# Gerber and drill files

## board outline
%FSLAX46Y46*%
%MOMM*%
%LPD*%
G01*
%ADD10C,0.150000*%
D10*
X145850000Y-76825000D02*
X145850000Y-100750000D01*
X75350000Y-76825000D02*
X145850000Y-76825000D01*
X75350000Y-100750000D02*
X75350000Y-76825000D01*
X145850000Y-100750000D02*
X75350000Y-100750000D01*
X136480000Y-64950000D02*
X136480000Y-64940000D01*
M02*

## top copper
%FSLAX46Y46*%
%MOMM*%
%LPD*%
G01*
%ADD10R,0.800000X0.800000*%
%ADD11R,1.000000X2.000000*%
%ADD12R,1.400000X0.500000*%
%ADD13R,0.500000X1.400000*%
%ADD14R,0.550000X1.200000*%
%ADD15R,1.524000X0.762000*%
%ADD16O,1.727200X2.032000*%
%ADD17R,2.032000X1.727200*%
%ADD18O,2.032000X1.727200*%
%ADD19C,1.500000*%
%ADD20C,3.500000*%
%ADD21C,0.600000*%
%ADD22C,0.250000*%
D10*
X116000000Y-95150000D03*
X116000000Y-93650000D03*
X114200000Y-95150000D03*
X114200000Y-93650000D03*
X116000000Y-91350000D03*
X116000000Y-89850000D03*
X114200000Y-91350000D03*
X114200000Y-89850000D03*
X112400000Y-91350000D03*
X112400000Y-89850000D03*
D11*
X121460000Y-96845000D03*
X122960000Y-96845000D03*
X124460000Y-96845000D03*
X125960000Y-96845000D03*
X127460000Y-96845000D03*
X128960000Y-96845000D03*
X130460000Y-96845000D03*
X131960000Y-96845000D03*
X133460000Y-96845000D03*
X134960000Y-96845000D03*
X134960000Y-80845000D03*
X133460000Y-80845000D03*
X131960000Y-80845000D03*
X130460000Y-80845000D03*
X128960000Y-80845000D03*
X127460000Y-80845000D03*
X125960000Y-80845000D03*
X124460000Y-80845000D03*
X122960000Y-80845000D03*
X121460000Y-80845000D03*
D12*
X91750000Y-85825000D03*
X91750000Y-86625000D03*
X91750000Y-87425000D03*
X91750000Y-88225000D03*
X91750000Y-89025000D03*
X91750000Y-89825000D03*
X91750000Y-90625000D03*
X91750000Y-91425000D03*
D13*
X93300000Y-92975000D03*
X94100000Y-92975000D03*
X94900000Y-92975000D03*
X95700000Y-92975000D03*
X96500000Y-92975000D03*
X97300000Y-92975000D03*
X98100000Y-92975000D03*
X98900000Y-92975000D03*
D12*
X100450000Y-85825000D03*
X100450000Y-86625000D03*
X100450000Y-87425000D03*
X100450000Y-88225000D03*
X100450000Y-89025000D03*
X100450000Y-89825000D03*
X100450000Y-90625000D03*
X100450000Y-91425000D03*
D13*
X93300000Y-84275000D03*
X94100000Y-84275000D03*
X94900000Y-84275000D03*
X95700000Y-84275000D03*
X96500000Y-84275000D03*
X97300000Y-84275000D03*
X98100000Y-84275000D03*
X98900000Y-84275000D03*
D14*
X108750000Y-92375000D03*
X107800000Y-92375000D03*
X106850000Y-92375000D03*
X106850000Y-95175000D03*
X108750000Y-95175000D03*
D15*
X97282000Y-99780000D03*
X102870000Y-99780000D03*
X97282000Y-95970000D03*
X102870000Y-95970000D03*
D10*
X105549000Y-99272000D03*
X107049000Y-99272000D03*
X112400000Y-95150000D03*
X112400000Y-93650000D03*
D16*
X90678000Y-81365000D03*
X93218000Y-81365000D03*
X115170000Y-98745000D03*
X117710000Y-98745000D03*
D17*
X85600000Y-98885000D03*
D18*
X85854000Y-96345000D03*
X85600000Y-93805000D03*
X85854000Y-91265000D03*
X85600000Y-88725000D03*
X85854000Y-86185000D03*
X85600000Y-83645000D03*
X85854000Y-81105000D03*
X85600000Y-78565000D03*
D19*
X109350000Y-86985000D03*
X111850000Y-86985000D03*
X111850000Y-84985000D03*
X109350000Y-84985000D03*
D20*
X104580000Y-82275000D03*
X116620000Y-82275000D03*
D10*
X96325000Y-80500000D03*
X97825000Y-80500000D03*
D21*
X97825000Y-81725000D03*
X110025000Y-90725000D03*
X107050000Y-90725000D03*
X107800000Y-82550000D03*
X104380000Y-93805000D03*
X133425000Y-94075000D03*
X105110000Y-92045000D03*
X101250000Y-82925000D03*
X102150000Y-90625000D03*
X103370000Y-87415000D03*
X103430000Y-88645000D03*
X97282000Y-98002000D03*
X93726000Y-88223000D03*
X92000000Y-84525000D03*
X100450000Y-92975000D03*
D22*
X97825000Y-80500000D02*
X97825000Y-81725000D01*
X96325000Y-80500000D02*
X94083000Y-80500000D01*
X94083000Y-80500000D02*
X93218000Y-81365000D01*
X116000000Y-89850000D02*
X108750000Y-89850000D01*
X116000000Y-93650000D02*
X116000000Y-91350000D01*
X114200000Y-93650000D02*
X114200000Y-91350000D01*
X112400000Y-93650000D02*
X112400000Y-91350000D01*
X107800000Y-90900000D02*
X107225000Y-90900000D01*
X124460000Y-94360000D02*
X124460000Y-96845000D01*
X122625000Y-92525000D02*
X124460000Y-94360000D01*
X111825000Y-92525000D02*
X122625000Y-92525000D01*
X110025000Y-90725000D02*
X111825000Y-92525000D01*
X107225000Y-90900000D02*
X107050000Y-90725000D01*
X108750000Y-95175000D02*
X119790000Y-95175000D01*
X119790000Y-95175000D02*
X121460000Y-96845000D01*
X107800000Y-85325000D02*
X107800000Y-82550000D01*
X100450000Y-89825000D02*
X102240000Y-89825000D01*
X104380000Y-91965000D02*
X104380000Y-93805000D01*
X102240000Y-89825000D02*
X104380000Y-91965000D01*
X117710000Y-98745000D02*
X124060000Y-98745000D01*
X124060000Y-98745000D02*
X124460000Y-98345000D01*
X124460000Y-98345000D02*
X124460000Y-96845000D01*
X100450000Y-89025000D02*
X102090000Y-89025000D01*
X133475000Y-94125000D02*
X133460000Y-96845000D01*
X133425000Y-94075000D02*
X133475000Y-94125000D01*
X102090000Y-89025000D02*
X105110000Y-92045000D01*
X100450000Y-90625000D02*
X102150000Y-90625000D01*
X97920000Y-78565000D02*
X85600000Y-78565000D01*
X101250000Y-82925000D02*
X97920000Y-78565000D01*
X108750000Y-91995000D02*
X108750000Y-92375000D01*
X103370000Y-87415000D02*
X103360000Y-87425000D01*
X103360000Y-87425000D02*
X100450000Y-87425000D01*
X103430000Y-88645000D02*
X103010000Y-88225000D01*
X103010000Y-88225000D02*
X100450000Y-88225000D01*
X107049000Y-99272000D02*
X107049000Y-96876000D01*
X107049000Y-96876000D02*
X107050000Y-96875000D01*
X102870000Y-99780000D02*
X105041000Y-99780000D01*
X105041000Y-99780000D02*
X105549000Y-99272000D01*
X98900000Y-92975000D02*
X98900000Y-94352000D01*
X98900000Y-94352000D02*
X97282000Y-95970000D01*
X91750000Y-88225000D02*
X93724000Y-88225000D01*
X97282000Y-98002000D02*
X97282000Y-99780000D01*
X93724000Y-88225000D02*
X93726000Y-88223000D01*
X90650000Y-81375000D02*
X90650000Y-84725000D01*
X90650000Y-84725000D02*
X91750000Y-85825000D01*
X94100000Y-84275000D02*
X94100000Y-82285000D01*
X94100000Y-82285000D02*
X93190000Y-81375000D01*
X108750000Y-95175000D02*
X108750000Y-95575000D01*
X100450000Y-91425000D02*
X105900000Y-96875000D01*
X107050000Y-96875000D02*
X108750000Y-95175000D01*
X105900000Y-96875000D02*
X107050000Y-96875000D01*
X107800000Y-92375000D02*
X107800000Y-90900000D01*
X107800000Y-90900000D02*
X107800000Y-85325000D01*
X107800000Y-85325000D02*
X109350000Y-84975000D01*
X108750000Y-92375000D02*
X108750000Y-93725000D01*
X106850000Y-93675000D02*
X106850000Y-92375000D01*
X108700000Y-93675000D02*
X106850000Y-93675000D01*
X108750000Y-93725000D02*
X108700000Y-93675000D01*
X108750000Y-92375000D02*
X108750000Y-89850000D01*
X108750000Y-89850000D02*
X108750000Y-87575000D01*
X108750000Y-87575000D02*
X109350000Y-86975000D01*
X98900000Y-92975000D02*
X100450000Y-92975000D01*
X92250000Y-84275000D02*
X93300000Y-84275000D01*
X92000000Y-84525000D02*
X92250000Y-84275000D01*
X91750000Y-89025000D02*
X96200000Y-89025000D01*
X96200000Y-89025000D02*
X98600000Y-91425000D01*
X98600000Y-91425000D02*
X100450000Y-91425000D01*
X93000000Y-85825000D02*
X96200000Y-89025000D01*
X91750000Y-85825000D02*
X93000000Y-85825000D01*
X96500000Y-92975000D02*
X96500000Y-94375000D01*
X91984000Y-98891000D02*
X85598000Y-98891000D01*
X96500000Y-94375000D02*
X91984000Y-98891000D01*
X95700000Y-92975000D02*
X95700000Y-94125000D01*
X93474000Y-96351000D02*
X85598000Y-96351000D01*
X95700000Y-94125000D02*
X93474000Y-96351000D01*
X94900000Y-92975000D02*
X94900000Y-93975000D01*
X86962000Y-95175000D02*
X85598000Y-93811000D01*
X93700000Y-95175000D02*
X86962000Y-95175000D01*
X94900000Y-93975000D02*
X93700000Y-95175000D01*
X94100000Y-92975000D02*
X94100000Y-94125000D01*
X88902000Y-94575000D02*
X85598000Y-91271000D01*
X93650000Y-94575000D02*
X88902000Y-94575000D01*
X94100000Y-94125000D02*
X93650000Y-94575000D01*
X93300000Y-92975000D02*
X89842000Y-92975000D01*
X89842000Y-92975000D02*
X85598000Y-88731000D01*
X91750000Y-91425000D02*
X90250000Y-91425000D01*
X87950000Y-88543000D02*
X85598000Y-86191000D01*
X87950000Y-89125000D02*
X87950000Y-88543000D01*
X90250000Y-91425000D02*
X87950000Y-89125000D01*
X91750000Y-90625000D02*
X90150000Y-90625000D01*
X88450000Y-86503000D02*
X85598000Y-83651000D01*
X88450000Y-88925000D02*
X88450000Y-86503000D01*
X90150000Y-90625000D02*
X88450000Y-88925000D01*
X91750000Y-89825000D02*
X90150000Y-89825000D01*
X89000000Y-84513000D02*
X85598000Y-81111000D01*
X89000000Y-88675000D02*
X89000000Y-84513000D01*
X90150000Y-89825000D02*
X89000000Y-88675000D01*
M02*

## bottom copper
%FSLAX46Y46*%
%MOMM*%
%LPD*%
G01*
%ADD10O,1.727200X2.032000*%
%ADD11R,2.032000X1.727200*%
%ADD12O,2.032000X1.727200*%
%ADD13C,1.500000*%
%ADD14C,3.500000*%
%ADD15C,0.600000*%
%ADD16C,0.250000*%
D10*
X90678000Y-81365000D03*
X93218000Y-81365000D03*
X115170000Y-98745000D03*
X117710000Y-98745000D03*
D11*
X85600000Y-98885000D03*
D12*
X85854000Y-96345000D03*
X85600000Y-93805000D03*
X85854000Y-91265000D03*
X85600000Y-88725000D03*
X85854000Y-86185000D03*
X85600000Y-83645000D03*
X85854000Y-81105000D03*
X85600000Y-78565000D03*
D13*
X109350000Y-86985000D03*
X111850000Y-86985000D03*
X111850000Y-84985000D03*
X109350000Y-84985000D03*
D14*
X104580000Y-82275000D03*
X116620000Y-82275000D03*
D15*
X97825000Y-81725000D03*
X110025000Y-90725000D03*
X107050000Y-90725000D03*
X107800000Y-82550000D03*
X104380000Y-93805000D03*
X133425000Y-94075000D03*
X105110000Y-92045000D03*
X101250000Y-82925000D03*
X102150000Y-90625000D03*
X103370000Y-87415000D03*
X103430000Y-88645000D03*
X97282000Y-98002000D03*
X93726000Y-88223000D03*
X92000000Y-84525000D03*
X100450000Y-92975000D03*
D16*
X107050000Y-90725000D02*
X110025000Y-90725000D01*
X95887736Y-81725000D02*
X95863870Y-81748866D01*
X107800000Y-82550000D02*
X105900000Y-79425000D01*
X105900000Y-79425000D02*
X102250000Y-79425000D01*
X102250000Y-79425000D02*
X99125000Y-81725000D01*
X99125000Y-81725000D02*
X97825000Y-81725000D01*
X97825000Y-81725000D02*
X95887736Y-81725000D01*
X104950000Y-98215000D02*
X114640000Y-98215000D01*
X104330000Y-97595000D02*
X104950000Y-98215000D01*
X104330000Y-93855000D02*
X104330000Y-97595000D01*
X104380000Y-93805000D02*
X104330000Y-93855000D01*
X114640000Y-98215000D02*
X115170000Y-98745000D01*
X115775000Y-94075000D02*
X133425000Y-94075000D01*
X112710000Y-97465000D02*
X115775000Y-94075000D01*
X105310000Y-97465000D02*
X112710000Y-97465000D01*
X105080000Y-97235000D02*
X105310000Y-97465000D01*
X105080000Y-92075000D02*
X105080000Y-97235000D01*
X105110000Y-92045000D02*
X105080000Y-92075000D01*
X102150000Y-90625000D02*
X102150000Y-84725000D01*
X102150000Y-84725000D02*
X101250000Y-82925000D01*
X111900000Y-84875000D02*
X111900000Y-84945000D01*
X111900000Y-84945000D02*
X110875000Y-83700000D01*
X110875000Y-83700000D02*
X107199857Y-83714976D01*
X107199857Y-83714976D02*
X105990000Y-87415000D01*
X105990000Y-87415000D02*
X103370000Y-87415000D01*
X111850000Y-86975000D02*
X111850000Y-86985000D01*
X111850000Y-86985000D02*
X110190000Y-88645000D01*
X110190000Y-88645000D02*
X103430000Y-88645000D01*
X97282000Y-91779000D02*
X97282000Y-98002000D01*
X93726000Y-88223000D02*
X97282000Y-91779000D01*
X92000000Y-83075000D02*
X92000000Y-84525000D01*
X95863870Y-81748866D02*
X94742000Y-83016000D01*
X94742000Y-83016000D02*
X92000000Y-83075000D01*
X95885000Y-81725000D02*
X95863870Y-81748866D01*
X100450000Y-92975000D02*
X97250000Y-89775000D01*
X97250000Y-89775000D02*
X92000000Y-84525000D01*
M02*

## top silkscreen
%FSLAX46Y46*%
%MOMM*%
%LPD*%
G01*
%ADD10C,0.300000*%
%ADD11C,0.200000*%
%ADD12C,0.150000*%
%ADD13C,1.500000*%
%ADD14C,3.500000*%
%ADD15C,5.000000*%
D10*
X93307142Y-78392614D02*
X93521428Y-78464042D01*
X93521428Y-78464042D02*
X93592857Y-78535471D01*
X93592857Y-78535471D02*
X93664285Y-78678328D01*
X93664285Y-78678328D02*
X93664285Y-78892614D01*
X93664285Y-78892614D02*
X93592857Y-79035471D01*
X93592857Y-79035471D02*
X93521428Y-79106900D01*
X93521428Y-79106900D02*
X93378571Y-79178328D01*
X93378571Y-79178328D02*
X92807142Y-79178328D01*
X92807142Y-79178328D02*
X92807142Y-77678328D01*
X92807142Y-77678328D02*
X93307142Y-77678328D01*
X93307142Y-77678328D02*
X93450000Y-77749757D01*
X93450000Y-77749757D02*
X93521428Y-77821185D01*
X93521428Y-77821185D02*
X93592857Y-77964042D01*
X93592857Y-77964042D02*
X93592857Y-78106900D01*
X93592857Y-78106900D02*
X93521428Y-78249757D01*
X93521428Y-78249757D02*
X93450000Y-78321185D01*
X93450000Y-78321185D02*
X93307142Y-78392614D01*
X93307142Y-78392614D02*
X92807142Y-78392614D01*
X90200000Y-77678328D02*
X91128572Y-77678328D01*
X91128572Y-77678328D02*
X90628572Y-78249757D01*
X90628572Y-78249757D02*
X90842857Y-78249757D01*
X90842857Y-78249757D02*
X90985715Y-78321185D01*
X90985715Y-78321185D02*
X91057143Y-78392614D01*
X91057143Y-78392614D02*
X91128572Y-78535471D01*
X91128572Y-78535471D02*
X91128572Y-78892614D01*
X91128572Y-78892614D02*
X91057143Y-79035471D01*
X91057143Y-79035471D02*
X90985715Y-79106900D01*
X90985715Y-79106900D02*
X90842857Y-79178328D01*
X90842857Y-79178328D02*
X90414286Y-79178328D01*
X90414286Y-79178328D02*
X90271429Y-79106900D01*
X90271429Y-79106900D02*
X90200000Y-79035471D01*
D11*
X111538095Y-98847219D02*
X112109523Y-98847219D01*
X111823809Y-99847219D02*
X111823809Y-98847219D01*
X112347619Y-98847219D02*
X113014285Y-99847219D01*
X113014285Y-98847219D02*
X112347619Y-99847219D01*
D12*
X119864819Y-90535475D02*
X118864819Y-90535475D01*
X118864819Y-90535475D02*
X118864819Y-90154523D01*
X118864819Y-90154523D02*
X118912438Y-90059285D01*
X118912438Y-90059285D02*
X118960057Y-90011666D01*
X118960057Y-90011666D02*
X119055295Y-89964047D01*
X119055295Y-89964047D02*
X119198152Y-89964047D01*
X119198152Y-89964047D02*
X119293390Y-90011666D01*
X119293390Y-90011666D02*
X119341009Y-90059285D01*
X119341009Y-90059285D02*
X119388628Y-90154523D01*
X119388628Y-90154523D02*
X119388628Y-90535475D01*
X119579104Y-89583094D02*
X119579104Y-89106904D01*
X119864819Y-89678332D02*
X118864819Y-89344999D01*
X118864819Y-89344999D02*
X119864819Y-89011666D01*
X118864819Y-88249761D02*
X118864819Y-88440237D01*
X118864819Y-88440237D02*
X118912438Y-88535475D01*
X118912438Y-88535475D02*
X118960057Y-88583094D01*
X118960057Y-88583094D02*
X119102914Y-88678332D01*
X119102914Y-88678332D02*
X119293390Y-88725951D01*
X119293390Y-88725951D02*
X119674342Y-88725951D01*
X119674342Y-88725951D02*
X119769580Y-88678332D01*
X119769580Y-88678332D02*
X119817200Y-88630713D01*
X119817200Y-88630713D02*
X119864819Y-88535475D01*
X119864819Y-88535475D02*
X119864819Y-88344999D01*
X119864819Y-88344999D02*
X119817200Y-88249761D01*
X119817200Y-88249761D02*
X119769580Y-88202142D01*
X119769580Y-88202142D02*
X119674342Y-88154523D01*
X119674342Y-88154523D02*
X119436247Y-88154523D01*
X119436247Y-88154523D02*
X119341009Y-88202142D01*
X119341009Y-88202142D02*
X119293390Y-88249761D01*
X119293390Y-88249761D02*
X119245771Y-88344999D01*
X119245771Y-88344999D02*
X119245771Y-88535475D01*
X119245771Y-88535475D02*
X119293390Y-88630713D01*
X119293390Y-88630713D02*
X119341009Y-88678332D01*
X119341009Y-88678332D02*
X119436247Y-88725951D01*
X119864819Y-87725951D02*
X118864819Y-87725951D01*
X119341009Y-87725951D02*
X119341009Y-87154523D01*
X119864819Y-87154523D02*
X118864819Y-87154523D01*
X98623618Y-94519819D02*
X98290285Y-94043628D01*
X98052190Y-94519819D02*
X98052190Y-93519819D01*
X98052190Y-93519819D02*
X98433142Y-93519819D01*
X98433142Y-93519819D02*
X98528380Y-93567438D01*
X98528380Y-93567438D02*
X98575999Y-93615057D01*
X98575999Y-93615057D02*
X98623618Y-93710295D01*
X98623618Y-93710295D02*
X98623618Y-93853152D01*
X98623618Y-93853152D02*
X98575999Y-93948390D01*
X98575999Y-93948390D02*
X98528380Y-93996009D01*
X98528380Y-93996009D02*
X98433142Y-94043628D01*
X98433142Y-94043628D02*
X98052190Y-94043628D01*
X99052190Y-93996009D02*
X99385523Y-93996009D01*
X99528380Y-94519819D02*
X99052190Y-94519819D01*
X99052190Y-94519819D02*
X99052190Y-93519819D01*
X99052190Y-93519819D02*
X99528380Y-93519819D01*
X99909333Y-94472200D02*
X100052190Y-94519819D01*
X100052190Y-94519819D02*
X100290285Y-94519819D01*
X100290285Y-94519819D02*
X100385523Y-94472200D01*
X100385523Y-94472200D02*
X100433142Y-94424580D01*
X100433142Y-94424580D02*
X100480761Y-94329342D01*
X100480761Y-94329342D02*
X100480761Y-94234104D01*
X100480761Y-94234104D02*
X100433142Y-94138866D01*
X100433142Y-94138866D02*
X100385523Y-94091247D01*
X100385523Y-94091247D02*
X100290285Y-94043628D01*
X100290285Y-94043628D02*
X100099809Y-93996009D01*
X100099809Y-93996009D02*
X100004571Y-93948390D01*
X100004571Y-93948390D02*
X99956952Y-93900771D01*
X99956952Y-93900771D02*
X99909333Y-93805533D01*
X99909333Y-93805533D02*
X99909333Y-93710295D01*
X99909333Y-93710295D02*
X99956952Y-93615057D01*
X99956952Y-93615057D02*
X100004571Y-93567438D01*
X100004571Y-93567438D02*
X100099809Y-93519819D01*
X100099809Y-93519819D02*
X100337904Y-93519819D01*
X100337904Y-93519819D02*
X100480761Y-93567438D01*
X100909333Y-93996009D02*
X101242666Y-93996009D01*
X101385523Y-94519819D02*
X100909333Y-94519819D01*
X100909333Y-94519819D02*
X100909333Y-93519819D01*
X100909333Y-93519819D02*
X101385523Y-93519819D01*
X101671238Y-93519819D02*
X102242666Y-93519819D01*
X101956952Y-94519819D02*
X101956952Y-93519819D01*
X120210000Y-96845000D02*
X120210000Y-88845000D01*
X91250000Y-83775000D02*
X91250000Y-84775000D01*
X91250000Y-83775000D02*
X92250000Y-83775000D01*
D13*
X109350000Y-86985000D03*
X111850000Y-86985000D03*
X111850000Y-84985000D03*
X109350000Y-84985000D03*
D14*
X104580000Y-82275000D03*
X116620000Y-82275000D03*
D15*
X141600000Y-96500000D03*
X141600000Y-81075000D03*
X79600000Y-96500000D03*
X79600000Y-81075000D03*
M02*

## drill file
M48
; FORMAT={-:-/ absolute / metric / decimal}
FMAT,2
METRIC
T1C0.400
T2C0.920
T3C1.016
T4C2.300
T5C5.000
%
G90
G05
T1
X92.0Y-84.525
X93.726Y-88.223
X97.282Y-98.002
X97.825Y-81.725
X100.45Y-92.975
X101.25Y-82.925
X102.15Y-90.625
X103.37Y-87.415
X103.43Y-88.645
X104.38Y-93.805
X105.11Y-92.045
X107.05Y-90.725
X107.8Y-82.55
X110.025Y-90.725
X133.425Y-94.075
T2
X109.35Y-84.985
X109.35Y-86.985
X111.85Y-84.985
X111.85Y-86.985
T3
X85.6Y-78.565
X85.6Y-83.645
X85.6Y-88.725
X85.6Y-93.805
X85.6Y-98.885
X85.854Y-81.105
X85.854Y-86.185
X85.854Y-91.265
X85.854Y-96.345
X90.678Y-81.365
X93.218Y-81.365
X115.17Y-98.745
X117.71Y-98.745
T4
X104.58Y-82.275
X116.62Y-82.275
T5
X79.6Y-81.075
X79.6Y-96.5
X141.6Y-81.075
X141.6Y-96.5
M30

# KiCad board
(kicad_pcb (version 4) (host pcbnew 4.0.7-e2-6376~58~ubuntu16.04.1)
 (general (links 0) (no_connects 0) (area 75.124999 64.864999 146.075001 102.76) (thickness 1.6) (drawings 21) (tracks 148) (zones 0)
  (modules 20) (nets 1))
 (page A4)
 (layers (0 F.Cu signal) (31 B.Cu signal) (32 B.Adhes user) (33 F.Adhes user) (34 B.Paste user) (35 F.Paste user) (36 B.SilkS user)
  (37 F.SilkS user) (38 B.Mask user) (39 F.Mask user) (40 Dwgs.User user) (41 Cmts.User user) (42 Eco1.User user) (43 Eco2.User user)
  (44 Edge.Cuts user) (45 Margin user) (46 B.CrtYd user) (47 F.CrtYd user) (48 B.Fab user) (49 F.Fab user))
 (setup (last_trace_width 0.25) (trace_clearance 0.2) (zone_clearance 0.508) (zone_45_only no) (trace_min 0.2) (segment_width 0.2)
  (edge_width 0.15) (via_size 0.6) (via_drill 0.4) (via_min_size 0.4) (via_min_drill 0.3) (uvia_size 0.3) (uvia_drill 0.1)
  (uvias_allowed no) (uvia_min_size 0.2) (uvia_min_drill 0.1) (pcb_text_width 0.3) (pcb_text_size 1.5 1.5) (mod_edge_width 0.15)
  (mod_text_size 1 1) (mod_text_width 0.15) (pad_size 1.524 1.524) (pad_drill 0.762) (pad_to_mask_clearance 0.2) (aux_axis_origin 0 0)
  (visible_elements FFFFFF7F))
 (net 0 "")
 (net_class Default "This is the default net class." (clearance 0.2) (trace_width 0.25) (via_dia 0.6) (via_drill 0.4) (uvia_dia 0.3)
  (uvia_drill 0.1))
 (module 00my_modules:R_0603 (layer F.Cu) (at 116 94.4 90)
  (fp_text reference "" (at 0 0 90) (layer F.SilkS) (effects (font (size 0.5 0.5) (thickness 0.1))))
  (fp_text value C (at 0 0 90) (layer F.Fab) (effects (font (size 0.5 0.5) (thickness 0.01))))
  (pad 1 smd rect (at -0.75 0 90) (size 0.8 0.8) (layers F.Cu F.Paste F.Mask))
  (pad 2 smd rect (at 0.75 0 90) (size 0.8 0.8) (layers F.Cu F.Paste F.Mask)))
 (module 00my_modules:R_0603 (layer F.Cu) (at 114.2 94.4 90)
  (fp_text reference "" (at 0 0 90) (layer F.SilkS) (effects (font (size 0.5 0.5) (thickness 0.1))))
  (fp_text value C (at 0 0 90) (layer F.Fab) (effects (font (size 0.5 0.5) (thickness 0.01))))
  (pad 1 smd rect (at -0.75 0 90) (size 0.8 0.8) (layers F.Cu F.Paste F.Mask))
  (pad 2 smd rect (at 0.75 0 90) (size 0.8 0.8) (layers F.Cu F.Paste F.Mask)))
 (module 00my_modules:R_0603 (layer F.Cu) (at 116 90.6 90)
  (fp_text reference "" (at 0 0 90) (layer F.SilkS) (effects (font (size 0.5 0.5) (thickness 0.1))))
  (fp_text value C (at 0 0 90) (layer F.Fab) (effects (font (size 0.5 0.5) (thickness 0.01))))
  (pad 1 smd rect (at -0.75 0 90) (size 0.8 0.8) (layers F.Cu F.Paste F.Mask))
  (pad 2 smd rect (at 0.75 0 90) (size 0.8 0.8) (layers F.Cu F.Paste F.Mask)))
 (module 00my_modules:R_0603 (layer F.Cu) (at 114.2 90.6 90)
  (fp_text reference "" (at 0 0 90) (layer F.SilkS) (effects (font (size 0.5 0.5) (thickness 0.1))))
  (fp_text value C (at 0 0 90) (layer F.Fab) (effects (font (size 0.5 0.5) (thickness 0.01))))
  (pad 1 smd rect (at -0.75 0 90) (size 0.8 0.8) (layers F.Cu F.Paste F.Mask))
  (pad 2 smd rect (at 0.75 0 90) (size 0.8 0.8) (layers F.Cu F.Paste F.Mask)))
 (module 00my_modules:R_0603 (layer F.Cu) (at 112.4 90.6 90)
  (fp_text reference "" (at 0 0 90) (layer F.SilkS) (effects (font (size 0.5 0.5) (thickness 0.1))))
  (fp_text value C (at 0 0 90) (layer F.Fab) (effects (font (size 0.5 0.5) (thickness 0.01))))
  (pad 1 smd rect (at -0.75 0 90) (size 0.8 0.8) (layers F.Cu F.Paste F.Mask))
  (pad 2 smd rect (at 0.75 0 90) (size 0.8 0.8) (layers F.Cu F.Paste F.Mask)))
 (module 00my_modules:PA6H (layer F.Cu) (at 128.21 88.845 90)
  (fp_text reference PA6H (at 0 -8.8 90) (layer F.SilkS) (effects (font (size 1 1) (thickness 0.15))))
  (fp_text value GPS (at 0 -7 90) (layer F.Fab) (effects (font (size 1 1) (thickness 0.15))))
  (fp_line (start -8 -8) (end 0 -8) (layer F.SilkS) (width 0.15))
  (pad VCC smd rect (at -8 -6.75 90) (size 2 1) (layers F.Cu F.Paste F.Mask))
  (pad 2 smd rect (at -8 -5.25 90) (size 2 1) (layers F.Cu F.Paste F.Mask))
  (pad GND smd rect (at -8 -3.75 90) (size 2 1) (layers F.Cu F.Paste F.Mask))
  (pad 4 smd rect (at -8 -2.25 90) (size 2 1) (layers F.Cu F.Paste F.Mask))
  (pad 5 smd rect (at -8 -0.75 90) (size 2 1) (layers F.Cu F.Paste F.Mask))
  (pad 6 smd rect (at -8 0.75 90) (size 2 1) (layers F.Cu F.Paste F.Mask))
  (pad 7 smd rect (at -8 2.25 90) (size 2 1) (layers F.Cu F.Paste F.Mask))
  (pad 8 smd rect (at -8 3.75 90) (size 2 1) (layers F.Cu F.Paste F.Mask))
  (pad TX smd rect (at -8 5.25 90) (size 2 1) (layers F.Cu F.Paste F.Mask))
  (pad RX smd rect (at -8 6.75 90) (size 2 1) (layers F.Cu F.Paste F.Mask))
  (pad 11 smd rect (at 8 6.75 90) (size 2 1) (layers F.Cu F.Paste F.Mask))
  (pad 12 smd rect (at 8 5.25 90) (size 2 1) (layers F.Cu F.Paste F.Mask))
  (pad 13 smd rect (at 8 3.75 90) (size 2 1) (layers F.Cu F.Paste F.Mask))
  (pad 14 smd rect (at 8 2.25 90) (size 2 1) (layers F.Cu F.Paste F.Mask))
  (pad 15 smd rect (at 8 0.75 90) (size 2 1) (layers F.Cu F.Paste F.Mask))
  (pad 16 smd rect (at 8 -0.75 90) (size 2 1) (layers F.Cu F.Paste F.Mask))
  (pad 17 smd rect (at 8 -2.25 90) (size 2 1) (layers F.Cu F.Paste F.Mask))
  (pad 18 smd rect (at 8 -3.75 90) (size 2 1) (layers F.Cu F.Paste F.Mask))
  (pad 19 smd rect (at 8 -5.25 90) (size 2 1) (layers F.Cu F.Paste F.Mask))
  (pad 20 smd rect (at 8 -6.75 90) (size 2 1) (layers F.Cu F.Paste F.Mask)))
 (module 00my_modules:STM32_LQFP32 (layer F.Cu) (at 96.1 88.625)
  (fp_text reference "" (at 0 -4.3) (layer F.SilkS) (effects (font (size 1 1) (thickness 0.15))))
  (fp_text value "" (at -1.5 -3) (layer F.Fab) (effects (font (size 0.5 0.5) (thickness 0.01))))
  (fp_line (start -4.85 -4.85) (end -4.85 -3.85) (layer F.SilkS) (width 0.15))
  (fp_line (start -4.85 -4.85) (end -3.85 -4.85) (layer F.SilkS) (width 0.15))
  (pad 3.3 smd rect (at -4.35 -2.8) (size 1.4 0.5) (layers F.Cu F.Paste F.Mask))
  (pad PF0 smd rect (at -4.35 -2) (size 1.4 0.5) (layers F.Cu F.Paste F.Mask))
  (pad PF1 smd rect (at -4.35 -1.2) (size 1.4 0.5) (layers F.Cu F.Paste F.Mask))
  (pad RST smd rect (at -4.35 -0.4) (size 1.4 0.5) (layers F.Cu F.Paste F.Mask))
  (pad 3.3 smd rect (at -4.35 0.4) (size 1.4 0.5) (layers F.Cu F.Paste F.Mask))
  (pad PA0 smd rect (at -4.35 1.2) (size 1.4 0.5) (layers F.Cu F.Paste F.Mask))
  (pad PA1 smd rect (at -4.35 2) (size 1.4 0.5) (layers F.Cu F.Paste F.Mask))
  (pad PA2 smd rect (at -4.35 2.8) (size 1.4 0.5) (layers F.Cu F.Paste F.Mask))
  (pad PA3 smd rect (at -2.8 4.35 90) (size 1.4 0.5) (layers F.Cu F.Paste F.Mask))
  (pad PA4 smd rect (at -2 4.35 90) (size 1.4 0.5) (layers F.Cu F.Paste F.Mask))
  (pad PA5 smd rect (at -1.2 4.35 90) (size 1.4 0.5) (layers F.Cu F.Paste F.Mask))
  (pad PA6 smd rect (at -0.4 4.35 90) (size 1.4 0.5) (layers F.Cu F.Paste F.Mask))
  (pad PA7 smd rect (at 0.4 4.35 90) (size 1.4 0.5) (layers F.Cu F.Paste F.Mask))
  (pad PB0 smd rect (at 1.2 4.35 90) (size 1.4 0.5) (layers F.Cu F.Paste F.Mask))
  (pad PB1 smd rect (at 2 4.35 90) (size 1.4 0.5) (layers F.Cu F.Paste F.Mask))
  (pad GND smd rect (at 2.8 4.35 90) (size 1.4 0.5) (layers F.Cu F.Paste F.Mask))
  (pad PA14 smd rect (at 4.35 -2.8) (size 1.4 0.5) (layers F.Cu F.Paste F.Mask))
  (pad PA13 smd rect (at 4.35 -2) (size 1.4 0.5) (layers F.Cu F.Paste F.Mask))
  (pad PA12 smd rect (at 4.35 -1.2) (size 1.4 0.5) (layers F.Cu F.Paste F.Mask))
  (pad PA11 smd rect (at 4.35 -0.4) (size 1.4 0.5) (layers F.Cu F.Paste F.Mask))
  (pad PA10 smd rect (at 4.35 0.4) (size 1.4 0.5) (layers F.Cu F.Paste F.Mask))
  (pad PA9 smd rect (at 4.35 1.2) (size 1.4 0.5) (layers F.Cu F.Paste F.Mask))
  (pad PA8 smd rect (at 4.35 2) (size 1.4 0.5) (layers F.Cu F.Paste F.Mask))
  (pad 3.3 smd rect (at 4.35 2.8) (size 1.4 0.5) (layers F.Cu F.Paste F.Mask))
  (pad GND smd rect (at -2.8 -4.35 90) (size 1.4 0.5) (layers F.Cu F.Paste F.Mask))
  (pad BOOT smd rect (at -2 -4.35 90) (size 1.4 0.5) (layers F.Cu F.Paste F.Mask))
  (pad PB7 smd rect (at -1.2 -4.35 90) (size 1.4 0.5) (layers F.Cu F.Paste F.Mask))
  (pad PB6 smd rect (at -0.4 -4.35 90) (size 1.4 0.5) (layers F.Cu F.Paste F.Mask))
  (pad PB5 smd rect (at 0.4 -4.35 90) (size 1.4 0.5) (layers F.Cu F.Paste F.Mask))
  (pad PB4 smd rect (at 1.2 -4.35 90) (size 1.4 0.5) (layers F.Cu F.Paste F.Mask))
  (pad PB3 smd rect (at 2 -4.35 90) (size 1.4 0.5) (layers F.Cu F.Paste F.Mask))
  (pad PA15 smd rect (at 2.8 -4.35 90) (size 1.4 0.5) (layers F.Cu F.Paste F.Mask)))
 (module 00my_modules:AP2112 (layer F.Cu) (at 107.8 93.775 270)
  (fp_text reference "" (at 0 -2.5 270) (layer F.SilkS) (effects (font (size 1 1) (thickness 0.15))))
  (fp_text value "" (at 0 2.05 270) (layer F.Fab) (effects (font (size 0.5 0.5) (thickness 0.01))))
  (pad VIN smd rect (at -1.4 -0.95 270) (size 1.2 0.55) (layers F.Cu F.Paste F.Mask))
  (pad GND smd rect (at -1.4 0 270) (size 1.2 0.55) (layers F.Cu F.Paste F.Mask))
  (pad EN smd rect (at -1.4 0.95 270) (size 1.2 0.55) (layers F.Cu F.Paste F.Mask))
  (pad NC smd rect (at 1.4 0.95 270) (size 1.2 0.55) (layers F.Cu F.Paste F.Mask))
  (pad VOUT smd rect (at 1.4 -0.95 270) (size 1.2 0.55) (layers F.Cu F.Paste F.Mask)))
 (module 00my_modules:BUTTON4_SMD (layer F.Cu) (at 100.076 97.875)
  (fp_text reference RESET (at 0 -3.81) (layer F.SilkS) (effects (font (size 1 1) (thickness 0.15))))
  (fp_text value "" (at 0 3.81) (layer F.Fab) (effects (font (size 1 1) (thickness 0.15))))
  (pad 1 smd rect (at -2.794 1.905) (size 1.524 0.762) (layers F.Cu F.Paste F.Mask))
  (pad 2 smd rect (at 2.794 1.905) (size 1.524 0.762) (layers F.Cu F.Paste F.Mask))
  (pad 3 smd rect (at -2.794 -1.905) (size 1.524 0.762) (layers F.Cu F.Paste F.Mask))
  (pad 4 smd rect (at 2.794 -1.905) (size 1.524 0.762) (layers F.Cu F.Paste F.Mask)))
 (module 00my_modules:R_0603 (layer F.Cu) (at 106.299 99.272)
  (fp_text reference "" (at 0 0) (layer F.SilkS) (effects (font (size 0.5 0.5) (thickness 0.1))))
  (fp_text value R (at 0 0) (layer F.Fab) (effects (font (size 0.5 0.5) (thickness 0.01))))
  (pad 1 smd rect (at -0.75 0) (size 0.8 0.8) (layers F.Cu F.Paste F.Mask))
  (pad 2 smd rect (at 0.75 0) (size 0.8 0.8) (layers F.Cu F.Paste F.Mask)))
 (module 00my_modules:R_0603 (layer F.Cu) (at 112.4 94.4 90)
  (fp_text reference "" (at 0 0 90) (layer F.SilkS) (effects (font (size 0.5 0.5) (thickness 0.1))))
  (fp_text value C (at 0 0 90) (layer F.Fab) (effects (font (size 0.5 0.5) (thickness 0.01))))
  (pad 1 smd rect (at -0.75 0 90) (size 0.8 0.8) (layers F.Cu F.Paste F.Mask))
  (pad 2 smd rect (at 0.75 0 90) (size 0.8 0.8) (layers F.Cu F.Paste F.Mask)))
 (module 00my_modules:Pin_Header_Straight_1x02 (layer B.Cu) (at 90.678 81.365 270)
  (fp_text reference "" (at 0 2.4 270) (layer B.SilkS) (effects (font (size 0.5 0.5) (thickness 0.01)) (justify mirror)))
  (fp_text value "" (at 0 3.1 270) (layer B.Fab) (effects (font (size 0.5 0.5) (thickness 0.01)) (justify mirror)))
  (pad 1 thru_hole oval (at 0 0 270) (size 2.032 1.7272) (drill 1.016) (layers *.Cu *.Mask B.SilkS))
  (pad 2 thru_hole oval (at 0 -2.54 270) (size 2.032 1.7272) (drill 1.016) (layers *.Cu *.Mask B.SilkS)))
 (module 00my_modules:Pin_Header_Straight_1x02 (layer B.Cu) (at 115.17 98.745 270)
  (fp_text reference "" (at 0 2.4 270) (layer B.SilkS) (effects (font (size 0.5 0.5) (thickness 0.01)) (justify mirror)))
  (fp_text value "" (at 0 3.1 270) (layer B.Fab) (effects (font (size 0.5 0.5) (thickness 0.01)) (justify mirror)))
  (pad 1 thru_hole oval (at 0 0 270) (size 2.032 1.7272) (drill 1.016) (layers *.Cu *.Mask B.SilkS))
  (pad 2 thru_hole oval (at 0 -2.54 270) (size 2.032 1.7272) (drill 1.016) (layers *.Cu *.Mask B.SilkS)))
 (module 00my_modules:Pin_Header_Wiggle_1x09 (layer B.Cu) (at 85.6 98.885)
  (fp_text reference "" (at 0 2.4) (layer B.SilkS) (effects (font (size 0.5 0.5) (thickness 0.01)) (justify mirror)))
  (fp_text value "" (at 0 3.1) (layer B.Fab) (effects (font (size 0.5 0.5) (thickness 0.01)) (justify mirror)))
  (pad 1 thru_hole rect (at 0 0) (size 2.032 1.7272) (drill 1.016) (layers *.Cu *.Mask B.SilkS))
  (pad 2 thru_hole oval (at 0.254 -2.54) (size 2.032 1.7272) (drill 1.016) (layers *.Cu *.Mask B.SilkS))
  (pad 3 thru_hole oval (at 0 -5.08) (size 2.032 1.7272) (drill 1.016) (layers *.Cu *.Mask B.SilkS))
  (pad 4 thru_hole oval (at 0.254 -7.62) (size 2.032 1.7272) (drill 1.016) (layers *.Cu *.Mask B.SilkS))
  (pad 5 thru_hole oval (at 0 -10.16) (size 2.032 1.7272) (drill 1.016) (layers *.Cu *.Mask B.SilkS))
  (pad 6 thru_hole oval (at 0.254 -12.7) (size 2.032 1.7272) (drill 1.016) (layers *.Cu *.Mask B.SilkS))
  (pad 7 thru_hole oval (at 0 -15.24) (size 2.032 1.7272) (drill 1.016) (layers *.Cu *.Mask B.SilkS))
  (pad 8 thru_hole oval (at 0.254 -17.78) (size 2.032 1.7272) (drill 1.016) (layers *.Cu *.Mask B.SilkS))
  (pad 9 thru_hole oval (at 0 -20.32) (size 2.032 1.7272) (drill 1.016) (layers *.Cu *.Mask B.SilkS)))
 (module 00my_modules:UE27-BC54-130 (layer F.Cu) (at 110.6 82.275 180)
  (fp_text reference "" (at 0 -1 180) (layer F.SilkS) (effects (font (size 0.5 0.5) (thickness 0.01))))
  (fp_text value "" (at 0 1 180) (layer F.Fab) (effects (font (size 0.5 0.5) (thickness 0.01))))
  (pad V thru_hole circle (at 1.25 -4.71 180) (size 1.5 1.5) (drill 0.92) (layers *.Cu *.Mask F.SilkS))
  (pad - thru_hole circle (at -1.25 -4.71 180) (size 1.5 1.5) (drill 0.92) (layers *.Cu *.Mask F.SilkS))
  (pad + thru_hole circle (at -1.25 -2.71 180) (size 1.5 1.5) (drill 0.92) (layers *.Cu *.Mask F.SilkS))
  (pad G thru_hole circle (at 1.25 -2.71 180) (size 1.5 1.5) (drill 0.92) (layers *.Cu *.Mask F.SilkS))
  (pad X thru_hole circle (at 6.02 0 180) (size 3.5 3.5) (drill 2.3) (layers *.Cu *.Mask F.SilkS))
  (pad X thru_hole circle (at -6.02 0 180) (size 3.5 3.5) (drill 2.3) (layers *.Cu *.Mask F.SilkS)))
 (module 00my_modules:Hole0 (layer F.Cu) (at 141.6 96.5)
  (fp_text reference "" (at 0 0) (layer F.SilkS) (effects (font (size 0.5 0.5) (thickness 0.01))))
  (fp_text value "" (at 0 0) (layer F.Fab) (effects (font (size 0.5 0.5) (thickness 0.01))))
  (pad "" np_thru_hole circle (at 0 0) (size 5 5) (drill 5) (layers *.Cu *.Mask F.SilkS)))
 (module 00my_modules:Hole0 (layer F.Cu) (at 141.6 81.075)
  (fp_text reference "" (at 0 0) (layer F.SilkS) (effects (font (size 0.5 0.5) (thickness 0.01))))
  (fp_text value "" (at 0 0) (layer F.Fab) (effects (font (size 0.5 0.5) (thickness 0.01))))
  (pad "" np_thru_hole circle (at 0 0) (size 5 5) (drill 5) (layers *.Cu *.Mask F.SilkS)))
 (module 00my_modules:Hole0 (layer F.Cu) (at 79.6 96.5)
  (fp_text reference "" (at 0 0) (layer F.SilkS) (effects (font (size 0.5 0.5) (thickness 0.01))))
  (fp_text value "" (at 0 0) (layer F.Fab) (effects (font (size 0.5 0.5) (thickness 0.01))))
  (pad "" np_thru_hole circle (at 0 0) (size 5 5) (drill 5) (layers *.Cu *.Mask F.SilkS)))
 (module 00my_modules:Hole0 (layer F.Cu) (at 79.6 81.075)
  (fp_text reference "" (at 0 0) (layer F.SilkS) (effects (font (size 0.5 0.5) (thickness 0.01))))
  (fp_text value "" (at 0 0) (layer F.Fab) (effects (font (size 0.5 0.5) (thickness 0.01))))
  (pad "" np_thru_hole circle (at 0 0) (size 5 5) (drill 5) (layers *.Cu *.Mask F.SilkS)))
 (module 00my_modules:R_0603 (layer F.Cu) (at 97.075 80.5)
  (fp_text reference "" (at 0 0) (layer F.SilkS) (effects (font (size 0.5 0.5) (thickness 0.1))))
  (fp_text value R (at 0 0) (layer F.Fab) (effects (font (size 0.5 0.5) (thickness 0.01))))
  (pad 1 smd rect (at -0.75 0) (size 0.8 0.8) (layers F.Cu F.Paste F.Mask))
  (pad 2 smd rect (at 0.75 0) (size 0.8 0.8) (layers F.Cu F.Paste F.Mask)))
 (gr_line (start 145.85 76.825) (end 145.85 100.75) (angle 90) (layer Edge.Cuts) (width 0.15))
 (gr_line (start 75.35 76.825) (end 145.85 76.825) (angle 90) (layer Edge.Cuts) (width 0.15))
 (gr_line (start 75.35 100.75) (end 75.35 76.825) (angle 90) (layer Edge.Cuts) (width 0.15))
 (gr_line (start 145.85 100.75) (end 75.35 100.75) (angle 90) (layer Edge.Cuts) (width 0.15))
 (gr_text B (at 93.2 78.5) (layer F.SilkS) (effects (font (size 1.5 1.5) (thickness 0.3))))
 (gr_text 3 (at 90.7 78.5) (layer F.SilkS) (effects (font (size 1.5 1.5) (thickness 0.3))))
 (gr_line (start 136.48 64.95) (end 136.48 64.94) (angle 90) (layer Edge.Cuts) (width 0.15))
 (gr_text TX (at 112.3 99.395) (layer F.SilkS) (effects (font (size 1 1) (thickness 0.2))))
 (segment (start 97.825 80.5) (end 97.825 81.725) (width 0.25) (layer F.Cu) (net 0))
 (via (at 97.825 81.725) (size 0.6) (drill 0.4) (layers F.Cu B.Cu) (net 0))
 (segment (start 96.325 80.5) (end 94.083 80.5) (width 0.25) (layer F.Cu) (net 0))
 (segment (start 94.083 80.5) (end 93.218 81.365) (width 0.25) (layer F.Cu) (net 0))
 (segment (start 116 89.85) (end 108.75 89.85) (width 0.25) (layer F.Cu) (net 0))
 (segment (start 116 93.65) (end 116 91.35) (width 0.25) (layer F.Cu) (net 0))
 (segment (start 114.2 93.65) (end 114.2 91.35) (width 0.25) (layer F.Cu) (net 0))
 (segment (start 112.4 93.65) (end 112.4 91.35) (width 0.25) (layer F.Cu) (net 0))
 (segment (start 107.8 90.9) (end 107.225 90.9) (width 0.25) (layer F.Cu) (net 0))
 (segment (start 124.46 94.36) (end 124.46 96.845) (width 0.25) (layer F.Cu) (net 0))
 (segment (start 122.625 92.525) (end 124.46 94.36) (width 0.25) (layer F.Cu) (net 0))
 (segment (start 111.825 92.525) (end 122.625 92.525) (width 0.25) (layer F.Cu) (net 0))
 (segment (start 110.025 90.725) (end 111.825 92.525) (width 0.25) (layer F.Cu) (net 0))
 (via (at 110.025 90.725) (size 0.6) (drill 0.4) (layers F.Cu B.Cu) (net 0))
 (segment (start 107.05 90.725) (end 110.025 90.725) (width 0.25) (layer B.Cu) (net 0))
 (via (at 107.05 90.725) (size 0.6) (drill 0.4) (layers F.Cu B.Cu) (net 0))
 (segment (start 107.225 90.9) (end 107.05 90.725) (width 0.25) (layer F.Cu) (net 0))
 (segment (start 108.75 95.175) (end 119.79 95.175) (width 0.25) (layer F.Cu) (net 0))
 (segment (start 119.79 95.175) (end 121.46 96.845) (width 0.25) (layer F.Cu) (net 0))
 (segment (start 107.8 85.325) (end 107.8 82.55) (width 0.25) (layer F.Cu) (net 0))
 (segment (start 95.887736 81.725) (end 95.86387 81.748866) (width 0.25) (layer B.Cu) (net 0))
 (segment (start 107.8 82.55) (end 105.9 79.425) (width 0.25) (layer B.Cu) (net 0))
 (segment (start 105.9 79.425) (end 102.25 79.425) (width 0.25) (layer B.Cu) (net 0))
 (segment (start 102.25 79.425) (end 99.125 81.725) (width 0.25) (layer B.Cu) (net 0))
 (segment (start 99.125 81.725) (end 97.825 81.725) (width 0.25) (layer B.Cu) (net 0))
 (segment (start 97.825 81.725) (end 95.887736 81.725) (width 0.25) (layer B.Cu) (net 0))
 (via (at 107.8 82.55) (size 0.6) (drill 0.4) (layers F.Cu B.Cu) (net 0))
 (segment (start 100.45 89.825) (end 102.24 89.825) (width 0.25) (layer F.Cu) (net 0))
 (segment (start 104.95 98.215) (end 114.64 98.215) (width 0.25) (layer B.Cu) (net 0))
 (segment (start 104.33 97.595) (end 104.95 98.215) (width 0.25) (layer B.Cu) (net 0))
 (segment (start 104.33 93.855) (end 104.33 97.595) (width 0.25) (layer B.Cu) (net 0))
 (segment (start 104.38 93.805) (end 104.33 93.855) (width 0.25) (layer B.Cu) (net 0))
 (via (at 104.38 93.805) (size 0.6) (drill 0.4) (layers F.Cu B.Cu) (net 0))
 (segment (start 104.38 91.965) (end 104.38 93.805) (width 0.25) (layer F.Cu) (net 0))
 (segment (start 102.24 89.825) (end 104.38 91.965) (width 0.25) (layer F.Cu) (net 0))
 (segment (start 114.64 98.215) (end 115.17 98.745) (width 0.25) (layer B.Cu) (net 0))
 (segment (start 117.71 98.745) (end 124.06 98.745) (width 0.25) (layer F.Cu) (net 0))
 (segment (start 124.06 98.745) (end 124.46 98.345) (width 0.25) (layer F.Cu) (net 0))
 (segment (start 124.46 98.345) (end 124.46 96.845) (width 0.25) (layer F.Cu) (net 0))
 (segment (start 100.45 89.025) (end 102.09 89.025) (width 0.25) (layer F.Cu) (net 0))
 (segment (start 133.475 94.125) (end 133.46 96.845) (width 0.25) (layer F.Cu) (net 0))
 (segment (start 133.425 94.075) (end 133.475 94.125) (width 0.25) (layer F.Cu) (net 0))
 (via (at 133.425 94.075) (size 0.6) (drill 0.4) (layers F.Cu B.Cu) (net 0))
 (segment (start 115.775 94.075) (end 133.425 94.075) (width 0.25) (layer B.Cu) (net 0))
 (segment (start 112.71 97.465) (end 115.775 94.075) (width 0.25) (layer B.Cu) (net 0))
 (segment (start 105.31 97.465) (end 112.71 97.465) (width 0.25) (layer B.Cu) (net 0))
 (segment (start 105.08 97.235) (end 105.31 97.465) (width 0.25) (layer B.Cu) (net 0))
 (segment (start 105.08 92.075) (end 105.08 97.235) (width 0.25) (layer B.Cu) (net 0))
 (segment (start 105.11 92.045) (end 105.08 92.075) (width 0.25) (layer B.Cu) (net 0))
 (via (at 105.11 92.045) (size 0.6) (drill 0.4) (layers F.Cu B.Cu) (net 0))
 (segment (start 102.09 89.025) (end 105.11 92.045) (width 0.25) (layer F.Cu) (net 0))
 (segment (start 100.45 90.625) (end 102.15 90.625) (width 0.25) (layer F.Cu) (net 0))
 (segment (start 97.92 78.565) (end 85.6 78.565) (width 0.25) (layer F.Cu) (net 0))
 (segment (start 101.25 82.925) (end 97.92 78.565) (width 0.25) (layer F.Cu) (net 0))
 (via (at 101.25 82.925) (size 0.6) (drill 0.4) (layers F.Cu B.Cu) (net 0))
 (segment (start 102.15 90.625) (end 102.15 84.725) (width 0.25) (layer B.Cu) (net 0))
 (segment (start 102.15 84.725) (end 101.25 82.925) (width 0.25) (layer B.Cu) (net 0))
 (via (at 102.15 90.625) (size 0.6) (drill 0.4) (layers F.Cu B.Cu) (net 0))
 (segment (start 108.75 91.995) (end 108.75 92.375) (width 0.25) (layer F.Cu) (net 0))
 (segment (start 111.9 84.875) (end 111.9 84.945) (width 0.25) (layer B.Cu) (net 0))
 (segment (start 111.9 84.945) (end 110.875 83.7) (width 0.25) (layer B.Cu) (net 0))
 (segment (start 110.875 83.7) (end 107.199857 83.714976) (width 0.25) (layer B.Cu) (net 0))
 (segment (start 107.199857 83.714976) (end 105.99 87.415) (width 0.25) (layer B.Cu) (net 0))
 (segment (start 105.99 87.415) (end 103.37 87.415) (width 0.25) (layer B.Cu) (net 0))
 (via (at 103.37 87.415) (size 0.6) (drill 0.4) (layers F.Cu B.Cu) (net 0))
 (segment (start 103.37 87.415) (end 103.36 87.425) (width 0.25) (layer F.Cu) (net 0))
 (segment (start 103.36 87.425) (end 100.45 87.425) (width 0.25) (layer F.Cu) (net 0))
 (segment (start 111.85 86.975) (end 111.85 86.985) (width 0.25) (layer B.Cu) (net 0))
 (segment (start 111.85 86.985) (end 110.19 88.645) (width 0.25) (layer B.Cu) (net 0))
 (segment (start 110.19 88.645) (end 103.43 88.645) (width 0.25) (layer B.Cu) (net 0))
 (via (at 103.43 88.645) (size 0.6) (drill 0.4) (layers F.Cu B.Cu) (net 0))
 (segment (start 103.43 88.645) (end 103.01 88.225) (width 0.25) (layer F.Cu) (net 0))
 (segment (start 103.01 88.225) (end 100.45 88.225) (width 0.25) (layer F.Cu) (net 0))
 (segment (start 107.049 99.272) (end 107.049 96.876) (width 0.25) (layer F.Cu) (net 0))
 (segment (start 107.049 96.876) (end 107.05 96.875) (width 0.25) (layer F.Cu) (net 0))
 (segment (start 102.87 99.78) (end 105.041 99.78) (width 0.25) (layer F.Cu) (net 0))
 (segment (start 105.041 99.78) (end 105.549 99.272) (width 0.25) (layer F.Cu) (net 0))
 (segment (start 98.9 92.975) (end 98.9 94.352) (width 0.25) (layer F.Cu) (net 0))
 (segment (start 98.9 94.352) (end 97.282 95.97) (width 0.25) (layer F.Cu) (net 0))
 (segment (start 91.75 88.225) (end 93.724 88.225) (width 0.25) (layer F.Cu) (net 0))
 (segment (start 97.282 98.002) (end 97.282 99.78) (width 0.25) (layer F.Cu) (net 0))
 (via (at 97.282 98.002) (size 0.6) (drill 0.4) (layers F.Cu B.Cu) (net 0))
 (segment (start 97.282 91.779) (end 97.282 98.002) (width 0.25) (layer B.Cu) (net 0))
 (segment (start 93.726 88.223) (end 97.282 91.779) (width 0.25) (layer B.Cu) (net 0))
 (via (at 93.726 88.223) (size 0.6) (drill 0.4) (layers F.Cu B.Cu) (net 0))
 (segment (start 93.724 88.225) (end 93.726 88.223) (width 0.25) (layer F.Cu) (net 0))
 (segment (start 90.65 81.375) (end 90.65 84.725) (width 0.25) (layer F.Cu) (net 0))
 (segment (start 90.65 84.725) (end 91.75 85.825) (width 0.25) (layer F.Cu) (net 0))
 (segment (start 94.1 84.275) (end 94.1 82.285) (width 0.25) (layer F.Cu) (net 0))
 (segment (start 94.1 82.285) (end 93.19 81.375) (width 0.25) (layer F.Cu) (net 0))
 (segment (start 108.75 95.175) (end 108.75 95.575) (width 0.25) (layer F.Cu) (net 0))
 (segment (start 100.45 91.425) (end 105.9 96.875) (width 0.25) (layer F.Cu) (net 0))
 (segment (start 107.05 96.875) (end 108.75 95.175) (width 0.25) (layer F.Cu) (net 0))
 (segment (start 105.9 96.875) (end 107.05 96.875) (width 0.25) (layer F.Cu) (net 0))
 (segment (start 107.8 92.375) (end 107.8 90.9) (width 0.25) (layer F.Cu) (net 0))
 (segment (start 107.8 90.9) (end 107.8 85.325) (width 0.25) (layer F.Cu) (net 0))
 (segment (start 107.8 85.325) (end 109.35 84.975) (width 0.25) (layer F.Cu) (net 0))
 (segment (start 108.75 92.375) (end 108.75 93.725) (width 0.25) (layer F.Cu) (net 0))
 (segment (start 106.85 93.675) (end 106.85 92.375) (width 0.25) (layer F.Cu) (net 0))
 (segment (start 108.7 93.675) (end 106.85 93.675) (width 0.25) (layer F.Cu) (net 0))
 (segment (start 108.75 93.725) (end 108.7 93.675) (width 0.25) (layer F.Cu) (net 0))
 (segment (start 108.75 92.375) (end 108.75 89.85) (width 0.25) (layer F.Cu) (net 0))
 (segment (start 108.75 89.85) (end 108.75 87.575) (width 0.25) (layer F.Cu) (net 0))
 (segment (start 108.75 87.575) (end 109.35 86.975) (width 0.25) (layer F.Cu) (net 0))
 (segment (start 92 83.075) (end 92 84.525) (width 0.25) (layer B.Cu) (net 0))
 (segment (start 95.86387 81.748866) (end 94.742 83.016) (width 0.25) (layer B.Cu) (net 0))
 (segment (start 94.742 83.016) (end 92 83.075) (width 0.25) (layer B.Cu) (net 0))
 (segment (start 95.885 81.725) (end 95.86387 81.748866) (width 0.25) (layer B.Cu) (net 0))
 (segment (start 98.9 92.975) (end 100.45 92.975) (width 0.25) (layer F.Cu) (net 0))
 (segment (start 92.25 84.275) (end 93.3 84.275) (width 0.25) (layer F.Cu) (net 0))
 (segment (start 92 84.525) (end 92.25 84.275) (width 0.25) (layer F.Cu) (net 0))
 (via (at 92 84.525) (size 0.6) (drill 0.4) (layers F.Cu B.Cu) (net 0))
 (segment (start 100.45 92.975) (end 97.25 89.775) (width 0.25) (layer B.Cu) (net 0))
 (segment (start 97.25 89.775) (end 92 84.525) (width 0.25) (layer B.Cu) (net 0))
 (via (at 100.45 92.975) (size 0.6) (drill 0.4) (layers F.Cu B.Cu) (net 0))
 (segment (start 91.75 89.025) (end 96.2 89.025) (width 0.25) (layer F.Cu) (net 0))
 (segment (start 96.2 89.025) (end 98.6 91.425) (width 0.25) (layer F.Cu) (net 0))
 (segment (start 98.6 91.425) (end 100.45 91.425) (width 0.25) (layer F.Cu) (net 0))
 (segment (start 93 85.825) (end 96.2 89.025) (width 0.25) (layer F.Cu) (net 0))
 (segment (start 91.75 85.825) (end 93 85.825) (width 0.25) (layer F.Cu) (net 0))
 (segment (start 96.5 92.975) (end 96.5 94.375) (width 0.25) (layer F.Cu) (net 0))
 (segment (start 91.984 98.891) (end 85.598 98.891) (width 0.25) (layer F.Cu) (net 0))
 (segment (start 96.5 94.375) (end 91.984 98.891) (width 0.25) (layer F.Cu) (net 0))
 (segment (start 95.7 92.975) (end 95.7 94.125) (width 0.25) (layer F.Cu) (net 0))
 (segment (start 93.474 96.351) (end 85.598 96.351) (width 0.25) (layer F.Cu) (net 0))
 (segment (start 95.7 94.125) (end 93.474 96.351) (width 0.25) (layer F.Cu) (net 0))
 (segment (start 94.9 92.975) (end 94.9 93.975) (width 0.25) (layer F.Cu) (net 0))
 (segment (start 86.962 95.175) (end 85.598 93.811) (width 0.25) (layer F.Cu) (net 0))
 (segment (start 93.7 95.175) (end 86.962 95.175) (width 0.25) (layer F.Cu) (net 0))
 (segment (start 94.9 93.975) (end 93.7 95.175) (width 0.25) (layer F.Cu) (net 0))
 (segment (start 94.1 92.975) (end 94.1 94.125) (width 0.25) (layer F.Cu) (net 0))
 (segment (start 88.902 94.575) (end 85.598 91.271) (width 0.25) (layer F.Cu) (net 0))
 (segment (start 93.65 94.575) (end 88.902 94.575) (width 0.25) (layer F.Cu) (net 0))
 (segment (start 94.1 94.125) (end 93.65 94.575) (width 0.25) (layer F.Cu) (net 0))
 (segment (start 93.3 92.975) (end 89.842 92.975) (width 0.25) (layer F.Cu) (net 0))
 (segment (start 89.842 92.975) (end 85.598 88.731) (width 0.25) (layer F.Cu) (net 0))
 (segment (start 91.75 91.425) (end 90.25 91.425) (width 0.25) (layer F.Cu) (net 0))
 (segment (start 87.95 88.543) (end 85.598 86.191) (width 0.25) (layer F.Cu) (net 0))
 (segment (start 87.95 89.125) (end 87.95 88.543) (width 0.25) (layer F.Cu) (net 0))
 (segment (start 90.25 91.425) (end 87.95 89.125) (width 0.25) (layer F.Cu) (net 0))
 (segment (start 91.75 90.625) (end 90.15 90.625) (width 0.25) (layer F.Cu) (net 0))
 (segment (start 88.45 86.503) (end 85.598 83.651) (width 0.25) (layer F.Cu) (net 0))
 (segment (start 88.45 88.925) (end 88.45 86.503) (width 0.25) (layer F.Cu) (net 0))
 (segment (start 90.15 90.625) (end 88.45 88.925) (width 0.25) (layer F.Cu) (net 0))
 (segment (start 91.75 89.825) (end 90.15 89.825) (width 0.25) (layer F.Cu) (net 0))
 (segment (start 89 84.513) (end 85.598 81.111) (width 0.25) (layer F.Cu) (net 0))
 (segment (start 89 88.675) (end 89 84.513) (width 0.25) (layer F.Cu) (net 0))
 (segment (start 90.15 89.825) (end 89 88.675) (width 0.25) (layer F.Cu) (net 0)))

